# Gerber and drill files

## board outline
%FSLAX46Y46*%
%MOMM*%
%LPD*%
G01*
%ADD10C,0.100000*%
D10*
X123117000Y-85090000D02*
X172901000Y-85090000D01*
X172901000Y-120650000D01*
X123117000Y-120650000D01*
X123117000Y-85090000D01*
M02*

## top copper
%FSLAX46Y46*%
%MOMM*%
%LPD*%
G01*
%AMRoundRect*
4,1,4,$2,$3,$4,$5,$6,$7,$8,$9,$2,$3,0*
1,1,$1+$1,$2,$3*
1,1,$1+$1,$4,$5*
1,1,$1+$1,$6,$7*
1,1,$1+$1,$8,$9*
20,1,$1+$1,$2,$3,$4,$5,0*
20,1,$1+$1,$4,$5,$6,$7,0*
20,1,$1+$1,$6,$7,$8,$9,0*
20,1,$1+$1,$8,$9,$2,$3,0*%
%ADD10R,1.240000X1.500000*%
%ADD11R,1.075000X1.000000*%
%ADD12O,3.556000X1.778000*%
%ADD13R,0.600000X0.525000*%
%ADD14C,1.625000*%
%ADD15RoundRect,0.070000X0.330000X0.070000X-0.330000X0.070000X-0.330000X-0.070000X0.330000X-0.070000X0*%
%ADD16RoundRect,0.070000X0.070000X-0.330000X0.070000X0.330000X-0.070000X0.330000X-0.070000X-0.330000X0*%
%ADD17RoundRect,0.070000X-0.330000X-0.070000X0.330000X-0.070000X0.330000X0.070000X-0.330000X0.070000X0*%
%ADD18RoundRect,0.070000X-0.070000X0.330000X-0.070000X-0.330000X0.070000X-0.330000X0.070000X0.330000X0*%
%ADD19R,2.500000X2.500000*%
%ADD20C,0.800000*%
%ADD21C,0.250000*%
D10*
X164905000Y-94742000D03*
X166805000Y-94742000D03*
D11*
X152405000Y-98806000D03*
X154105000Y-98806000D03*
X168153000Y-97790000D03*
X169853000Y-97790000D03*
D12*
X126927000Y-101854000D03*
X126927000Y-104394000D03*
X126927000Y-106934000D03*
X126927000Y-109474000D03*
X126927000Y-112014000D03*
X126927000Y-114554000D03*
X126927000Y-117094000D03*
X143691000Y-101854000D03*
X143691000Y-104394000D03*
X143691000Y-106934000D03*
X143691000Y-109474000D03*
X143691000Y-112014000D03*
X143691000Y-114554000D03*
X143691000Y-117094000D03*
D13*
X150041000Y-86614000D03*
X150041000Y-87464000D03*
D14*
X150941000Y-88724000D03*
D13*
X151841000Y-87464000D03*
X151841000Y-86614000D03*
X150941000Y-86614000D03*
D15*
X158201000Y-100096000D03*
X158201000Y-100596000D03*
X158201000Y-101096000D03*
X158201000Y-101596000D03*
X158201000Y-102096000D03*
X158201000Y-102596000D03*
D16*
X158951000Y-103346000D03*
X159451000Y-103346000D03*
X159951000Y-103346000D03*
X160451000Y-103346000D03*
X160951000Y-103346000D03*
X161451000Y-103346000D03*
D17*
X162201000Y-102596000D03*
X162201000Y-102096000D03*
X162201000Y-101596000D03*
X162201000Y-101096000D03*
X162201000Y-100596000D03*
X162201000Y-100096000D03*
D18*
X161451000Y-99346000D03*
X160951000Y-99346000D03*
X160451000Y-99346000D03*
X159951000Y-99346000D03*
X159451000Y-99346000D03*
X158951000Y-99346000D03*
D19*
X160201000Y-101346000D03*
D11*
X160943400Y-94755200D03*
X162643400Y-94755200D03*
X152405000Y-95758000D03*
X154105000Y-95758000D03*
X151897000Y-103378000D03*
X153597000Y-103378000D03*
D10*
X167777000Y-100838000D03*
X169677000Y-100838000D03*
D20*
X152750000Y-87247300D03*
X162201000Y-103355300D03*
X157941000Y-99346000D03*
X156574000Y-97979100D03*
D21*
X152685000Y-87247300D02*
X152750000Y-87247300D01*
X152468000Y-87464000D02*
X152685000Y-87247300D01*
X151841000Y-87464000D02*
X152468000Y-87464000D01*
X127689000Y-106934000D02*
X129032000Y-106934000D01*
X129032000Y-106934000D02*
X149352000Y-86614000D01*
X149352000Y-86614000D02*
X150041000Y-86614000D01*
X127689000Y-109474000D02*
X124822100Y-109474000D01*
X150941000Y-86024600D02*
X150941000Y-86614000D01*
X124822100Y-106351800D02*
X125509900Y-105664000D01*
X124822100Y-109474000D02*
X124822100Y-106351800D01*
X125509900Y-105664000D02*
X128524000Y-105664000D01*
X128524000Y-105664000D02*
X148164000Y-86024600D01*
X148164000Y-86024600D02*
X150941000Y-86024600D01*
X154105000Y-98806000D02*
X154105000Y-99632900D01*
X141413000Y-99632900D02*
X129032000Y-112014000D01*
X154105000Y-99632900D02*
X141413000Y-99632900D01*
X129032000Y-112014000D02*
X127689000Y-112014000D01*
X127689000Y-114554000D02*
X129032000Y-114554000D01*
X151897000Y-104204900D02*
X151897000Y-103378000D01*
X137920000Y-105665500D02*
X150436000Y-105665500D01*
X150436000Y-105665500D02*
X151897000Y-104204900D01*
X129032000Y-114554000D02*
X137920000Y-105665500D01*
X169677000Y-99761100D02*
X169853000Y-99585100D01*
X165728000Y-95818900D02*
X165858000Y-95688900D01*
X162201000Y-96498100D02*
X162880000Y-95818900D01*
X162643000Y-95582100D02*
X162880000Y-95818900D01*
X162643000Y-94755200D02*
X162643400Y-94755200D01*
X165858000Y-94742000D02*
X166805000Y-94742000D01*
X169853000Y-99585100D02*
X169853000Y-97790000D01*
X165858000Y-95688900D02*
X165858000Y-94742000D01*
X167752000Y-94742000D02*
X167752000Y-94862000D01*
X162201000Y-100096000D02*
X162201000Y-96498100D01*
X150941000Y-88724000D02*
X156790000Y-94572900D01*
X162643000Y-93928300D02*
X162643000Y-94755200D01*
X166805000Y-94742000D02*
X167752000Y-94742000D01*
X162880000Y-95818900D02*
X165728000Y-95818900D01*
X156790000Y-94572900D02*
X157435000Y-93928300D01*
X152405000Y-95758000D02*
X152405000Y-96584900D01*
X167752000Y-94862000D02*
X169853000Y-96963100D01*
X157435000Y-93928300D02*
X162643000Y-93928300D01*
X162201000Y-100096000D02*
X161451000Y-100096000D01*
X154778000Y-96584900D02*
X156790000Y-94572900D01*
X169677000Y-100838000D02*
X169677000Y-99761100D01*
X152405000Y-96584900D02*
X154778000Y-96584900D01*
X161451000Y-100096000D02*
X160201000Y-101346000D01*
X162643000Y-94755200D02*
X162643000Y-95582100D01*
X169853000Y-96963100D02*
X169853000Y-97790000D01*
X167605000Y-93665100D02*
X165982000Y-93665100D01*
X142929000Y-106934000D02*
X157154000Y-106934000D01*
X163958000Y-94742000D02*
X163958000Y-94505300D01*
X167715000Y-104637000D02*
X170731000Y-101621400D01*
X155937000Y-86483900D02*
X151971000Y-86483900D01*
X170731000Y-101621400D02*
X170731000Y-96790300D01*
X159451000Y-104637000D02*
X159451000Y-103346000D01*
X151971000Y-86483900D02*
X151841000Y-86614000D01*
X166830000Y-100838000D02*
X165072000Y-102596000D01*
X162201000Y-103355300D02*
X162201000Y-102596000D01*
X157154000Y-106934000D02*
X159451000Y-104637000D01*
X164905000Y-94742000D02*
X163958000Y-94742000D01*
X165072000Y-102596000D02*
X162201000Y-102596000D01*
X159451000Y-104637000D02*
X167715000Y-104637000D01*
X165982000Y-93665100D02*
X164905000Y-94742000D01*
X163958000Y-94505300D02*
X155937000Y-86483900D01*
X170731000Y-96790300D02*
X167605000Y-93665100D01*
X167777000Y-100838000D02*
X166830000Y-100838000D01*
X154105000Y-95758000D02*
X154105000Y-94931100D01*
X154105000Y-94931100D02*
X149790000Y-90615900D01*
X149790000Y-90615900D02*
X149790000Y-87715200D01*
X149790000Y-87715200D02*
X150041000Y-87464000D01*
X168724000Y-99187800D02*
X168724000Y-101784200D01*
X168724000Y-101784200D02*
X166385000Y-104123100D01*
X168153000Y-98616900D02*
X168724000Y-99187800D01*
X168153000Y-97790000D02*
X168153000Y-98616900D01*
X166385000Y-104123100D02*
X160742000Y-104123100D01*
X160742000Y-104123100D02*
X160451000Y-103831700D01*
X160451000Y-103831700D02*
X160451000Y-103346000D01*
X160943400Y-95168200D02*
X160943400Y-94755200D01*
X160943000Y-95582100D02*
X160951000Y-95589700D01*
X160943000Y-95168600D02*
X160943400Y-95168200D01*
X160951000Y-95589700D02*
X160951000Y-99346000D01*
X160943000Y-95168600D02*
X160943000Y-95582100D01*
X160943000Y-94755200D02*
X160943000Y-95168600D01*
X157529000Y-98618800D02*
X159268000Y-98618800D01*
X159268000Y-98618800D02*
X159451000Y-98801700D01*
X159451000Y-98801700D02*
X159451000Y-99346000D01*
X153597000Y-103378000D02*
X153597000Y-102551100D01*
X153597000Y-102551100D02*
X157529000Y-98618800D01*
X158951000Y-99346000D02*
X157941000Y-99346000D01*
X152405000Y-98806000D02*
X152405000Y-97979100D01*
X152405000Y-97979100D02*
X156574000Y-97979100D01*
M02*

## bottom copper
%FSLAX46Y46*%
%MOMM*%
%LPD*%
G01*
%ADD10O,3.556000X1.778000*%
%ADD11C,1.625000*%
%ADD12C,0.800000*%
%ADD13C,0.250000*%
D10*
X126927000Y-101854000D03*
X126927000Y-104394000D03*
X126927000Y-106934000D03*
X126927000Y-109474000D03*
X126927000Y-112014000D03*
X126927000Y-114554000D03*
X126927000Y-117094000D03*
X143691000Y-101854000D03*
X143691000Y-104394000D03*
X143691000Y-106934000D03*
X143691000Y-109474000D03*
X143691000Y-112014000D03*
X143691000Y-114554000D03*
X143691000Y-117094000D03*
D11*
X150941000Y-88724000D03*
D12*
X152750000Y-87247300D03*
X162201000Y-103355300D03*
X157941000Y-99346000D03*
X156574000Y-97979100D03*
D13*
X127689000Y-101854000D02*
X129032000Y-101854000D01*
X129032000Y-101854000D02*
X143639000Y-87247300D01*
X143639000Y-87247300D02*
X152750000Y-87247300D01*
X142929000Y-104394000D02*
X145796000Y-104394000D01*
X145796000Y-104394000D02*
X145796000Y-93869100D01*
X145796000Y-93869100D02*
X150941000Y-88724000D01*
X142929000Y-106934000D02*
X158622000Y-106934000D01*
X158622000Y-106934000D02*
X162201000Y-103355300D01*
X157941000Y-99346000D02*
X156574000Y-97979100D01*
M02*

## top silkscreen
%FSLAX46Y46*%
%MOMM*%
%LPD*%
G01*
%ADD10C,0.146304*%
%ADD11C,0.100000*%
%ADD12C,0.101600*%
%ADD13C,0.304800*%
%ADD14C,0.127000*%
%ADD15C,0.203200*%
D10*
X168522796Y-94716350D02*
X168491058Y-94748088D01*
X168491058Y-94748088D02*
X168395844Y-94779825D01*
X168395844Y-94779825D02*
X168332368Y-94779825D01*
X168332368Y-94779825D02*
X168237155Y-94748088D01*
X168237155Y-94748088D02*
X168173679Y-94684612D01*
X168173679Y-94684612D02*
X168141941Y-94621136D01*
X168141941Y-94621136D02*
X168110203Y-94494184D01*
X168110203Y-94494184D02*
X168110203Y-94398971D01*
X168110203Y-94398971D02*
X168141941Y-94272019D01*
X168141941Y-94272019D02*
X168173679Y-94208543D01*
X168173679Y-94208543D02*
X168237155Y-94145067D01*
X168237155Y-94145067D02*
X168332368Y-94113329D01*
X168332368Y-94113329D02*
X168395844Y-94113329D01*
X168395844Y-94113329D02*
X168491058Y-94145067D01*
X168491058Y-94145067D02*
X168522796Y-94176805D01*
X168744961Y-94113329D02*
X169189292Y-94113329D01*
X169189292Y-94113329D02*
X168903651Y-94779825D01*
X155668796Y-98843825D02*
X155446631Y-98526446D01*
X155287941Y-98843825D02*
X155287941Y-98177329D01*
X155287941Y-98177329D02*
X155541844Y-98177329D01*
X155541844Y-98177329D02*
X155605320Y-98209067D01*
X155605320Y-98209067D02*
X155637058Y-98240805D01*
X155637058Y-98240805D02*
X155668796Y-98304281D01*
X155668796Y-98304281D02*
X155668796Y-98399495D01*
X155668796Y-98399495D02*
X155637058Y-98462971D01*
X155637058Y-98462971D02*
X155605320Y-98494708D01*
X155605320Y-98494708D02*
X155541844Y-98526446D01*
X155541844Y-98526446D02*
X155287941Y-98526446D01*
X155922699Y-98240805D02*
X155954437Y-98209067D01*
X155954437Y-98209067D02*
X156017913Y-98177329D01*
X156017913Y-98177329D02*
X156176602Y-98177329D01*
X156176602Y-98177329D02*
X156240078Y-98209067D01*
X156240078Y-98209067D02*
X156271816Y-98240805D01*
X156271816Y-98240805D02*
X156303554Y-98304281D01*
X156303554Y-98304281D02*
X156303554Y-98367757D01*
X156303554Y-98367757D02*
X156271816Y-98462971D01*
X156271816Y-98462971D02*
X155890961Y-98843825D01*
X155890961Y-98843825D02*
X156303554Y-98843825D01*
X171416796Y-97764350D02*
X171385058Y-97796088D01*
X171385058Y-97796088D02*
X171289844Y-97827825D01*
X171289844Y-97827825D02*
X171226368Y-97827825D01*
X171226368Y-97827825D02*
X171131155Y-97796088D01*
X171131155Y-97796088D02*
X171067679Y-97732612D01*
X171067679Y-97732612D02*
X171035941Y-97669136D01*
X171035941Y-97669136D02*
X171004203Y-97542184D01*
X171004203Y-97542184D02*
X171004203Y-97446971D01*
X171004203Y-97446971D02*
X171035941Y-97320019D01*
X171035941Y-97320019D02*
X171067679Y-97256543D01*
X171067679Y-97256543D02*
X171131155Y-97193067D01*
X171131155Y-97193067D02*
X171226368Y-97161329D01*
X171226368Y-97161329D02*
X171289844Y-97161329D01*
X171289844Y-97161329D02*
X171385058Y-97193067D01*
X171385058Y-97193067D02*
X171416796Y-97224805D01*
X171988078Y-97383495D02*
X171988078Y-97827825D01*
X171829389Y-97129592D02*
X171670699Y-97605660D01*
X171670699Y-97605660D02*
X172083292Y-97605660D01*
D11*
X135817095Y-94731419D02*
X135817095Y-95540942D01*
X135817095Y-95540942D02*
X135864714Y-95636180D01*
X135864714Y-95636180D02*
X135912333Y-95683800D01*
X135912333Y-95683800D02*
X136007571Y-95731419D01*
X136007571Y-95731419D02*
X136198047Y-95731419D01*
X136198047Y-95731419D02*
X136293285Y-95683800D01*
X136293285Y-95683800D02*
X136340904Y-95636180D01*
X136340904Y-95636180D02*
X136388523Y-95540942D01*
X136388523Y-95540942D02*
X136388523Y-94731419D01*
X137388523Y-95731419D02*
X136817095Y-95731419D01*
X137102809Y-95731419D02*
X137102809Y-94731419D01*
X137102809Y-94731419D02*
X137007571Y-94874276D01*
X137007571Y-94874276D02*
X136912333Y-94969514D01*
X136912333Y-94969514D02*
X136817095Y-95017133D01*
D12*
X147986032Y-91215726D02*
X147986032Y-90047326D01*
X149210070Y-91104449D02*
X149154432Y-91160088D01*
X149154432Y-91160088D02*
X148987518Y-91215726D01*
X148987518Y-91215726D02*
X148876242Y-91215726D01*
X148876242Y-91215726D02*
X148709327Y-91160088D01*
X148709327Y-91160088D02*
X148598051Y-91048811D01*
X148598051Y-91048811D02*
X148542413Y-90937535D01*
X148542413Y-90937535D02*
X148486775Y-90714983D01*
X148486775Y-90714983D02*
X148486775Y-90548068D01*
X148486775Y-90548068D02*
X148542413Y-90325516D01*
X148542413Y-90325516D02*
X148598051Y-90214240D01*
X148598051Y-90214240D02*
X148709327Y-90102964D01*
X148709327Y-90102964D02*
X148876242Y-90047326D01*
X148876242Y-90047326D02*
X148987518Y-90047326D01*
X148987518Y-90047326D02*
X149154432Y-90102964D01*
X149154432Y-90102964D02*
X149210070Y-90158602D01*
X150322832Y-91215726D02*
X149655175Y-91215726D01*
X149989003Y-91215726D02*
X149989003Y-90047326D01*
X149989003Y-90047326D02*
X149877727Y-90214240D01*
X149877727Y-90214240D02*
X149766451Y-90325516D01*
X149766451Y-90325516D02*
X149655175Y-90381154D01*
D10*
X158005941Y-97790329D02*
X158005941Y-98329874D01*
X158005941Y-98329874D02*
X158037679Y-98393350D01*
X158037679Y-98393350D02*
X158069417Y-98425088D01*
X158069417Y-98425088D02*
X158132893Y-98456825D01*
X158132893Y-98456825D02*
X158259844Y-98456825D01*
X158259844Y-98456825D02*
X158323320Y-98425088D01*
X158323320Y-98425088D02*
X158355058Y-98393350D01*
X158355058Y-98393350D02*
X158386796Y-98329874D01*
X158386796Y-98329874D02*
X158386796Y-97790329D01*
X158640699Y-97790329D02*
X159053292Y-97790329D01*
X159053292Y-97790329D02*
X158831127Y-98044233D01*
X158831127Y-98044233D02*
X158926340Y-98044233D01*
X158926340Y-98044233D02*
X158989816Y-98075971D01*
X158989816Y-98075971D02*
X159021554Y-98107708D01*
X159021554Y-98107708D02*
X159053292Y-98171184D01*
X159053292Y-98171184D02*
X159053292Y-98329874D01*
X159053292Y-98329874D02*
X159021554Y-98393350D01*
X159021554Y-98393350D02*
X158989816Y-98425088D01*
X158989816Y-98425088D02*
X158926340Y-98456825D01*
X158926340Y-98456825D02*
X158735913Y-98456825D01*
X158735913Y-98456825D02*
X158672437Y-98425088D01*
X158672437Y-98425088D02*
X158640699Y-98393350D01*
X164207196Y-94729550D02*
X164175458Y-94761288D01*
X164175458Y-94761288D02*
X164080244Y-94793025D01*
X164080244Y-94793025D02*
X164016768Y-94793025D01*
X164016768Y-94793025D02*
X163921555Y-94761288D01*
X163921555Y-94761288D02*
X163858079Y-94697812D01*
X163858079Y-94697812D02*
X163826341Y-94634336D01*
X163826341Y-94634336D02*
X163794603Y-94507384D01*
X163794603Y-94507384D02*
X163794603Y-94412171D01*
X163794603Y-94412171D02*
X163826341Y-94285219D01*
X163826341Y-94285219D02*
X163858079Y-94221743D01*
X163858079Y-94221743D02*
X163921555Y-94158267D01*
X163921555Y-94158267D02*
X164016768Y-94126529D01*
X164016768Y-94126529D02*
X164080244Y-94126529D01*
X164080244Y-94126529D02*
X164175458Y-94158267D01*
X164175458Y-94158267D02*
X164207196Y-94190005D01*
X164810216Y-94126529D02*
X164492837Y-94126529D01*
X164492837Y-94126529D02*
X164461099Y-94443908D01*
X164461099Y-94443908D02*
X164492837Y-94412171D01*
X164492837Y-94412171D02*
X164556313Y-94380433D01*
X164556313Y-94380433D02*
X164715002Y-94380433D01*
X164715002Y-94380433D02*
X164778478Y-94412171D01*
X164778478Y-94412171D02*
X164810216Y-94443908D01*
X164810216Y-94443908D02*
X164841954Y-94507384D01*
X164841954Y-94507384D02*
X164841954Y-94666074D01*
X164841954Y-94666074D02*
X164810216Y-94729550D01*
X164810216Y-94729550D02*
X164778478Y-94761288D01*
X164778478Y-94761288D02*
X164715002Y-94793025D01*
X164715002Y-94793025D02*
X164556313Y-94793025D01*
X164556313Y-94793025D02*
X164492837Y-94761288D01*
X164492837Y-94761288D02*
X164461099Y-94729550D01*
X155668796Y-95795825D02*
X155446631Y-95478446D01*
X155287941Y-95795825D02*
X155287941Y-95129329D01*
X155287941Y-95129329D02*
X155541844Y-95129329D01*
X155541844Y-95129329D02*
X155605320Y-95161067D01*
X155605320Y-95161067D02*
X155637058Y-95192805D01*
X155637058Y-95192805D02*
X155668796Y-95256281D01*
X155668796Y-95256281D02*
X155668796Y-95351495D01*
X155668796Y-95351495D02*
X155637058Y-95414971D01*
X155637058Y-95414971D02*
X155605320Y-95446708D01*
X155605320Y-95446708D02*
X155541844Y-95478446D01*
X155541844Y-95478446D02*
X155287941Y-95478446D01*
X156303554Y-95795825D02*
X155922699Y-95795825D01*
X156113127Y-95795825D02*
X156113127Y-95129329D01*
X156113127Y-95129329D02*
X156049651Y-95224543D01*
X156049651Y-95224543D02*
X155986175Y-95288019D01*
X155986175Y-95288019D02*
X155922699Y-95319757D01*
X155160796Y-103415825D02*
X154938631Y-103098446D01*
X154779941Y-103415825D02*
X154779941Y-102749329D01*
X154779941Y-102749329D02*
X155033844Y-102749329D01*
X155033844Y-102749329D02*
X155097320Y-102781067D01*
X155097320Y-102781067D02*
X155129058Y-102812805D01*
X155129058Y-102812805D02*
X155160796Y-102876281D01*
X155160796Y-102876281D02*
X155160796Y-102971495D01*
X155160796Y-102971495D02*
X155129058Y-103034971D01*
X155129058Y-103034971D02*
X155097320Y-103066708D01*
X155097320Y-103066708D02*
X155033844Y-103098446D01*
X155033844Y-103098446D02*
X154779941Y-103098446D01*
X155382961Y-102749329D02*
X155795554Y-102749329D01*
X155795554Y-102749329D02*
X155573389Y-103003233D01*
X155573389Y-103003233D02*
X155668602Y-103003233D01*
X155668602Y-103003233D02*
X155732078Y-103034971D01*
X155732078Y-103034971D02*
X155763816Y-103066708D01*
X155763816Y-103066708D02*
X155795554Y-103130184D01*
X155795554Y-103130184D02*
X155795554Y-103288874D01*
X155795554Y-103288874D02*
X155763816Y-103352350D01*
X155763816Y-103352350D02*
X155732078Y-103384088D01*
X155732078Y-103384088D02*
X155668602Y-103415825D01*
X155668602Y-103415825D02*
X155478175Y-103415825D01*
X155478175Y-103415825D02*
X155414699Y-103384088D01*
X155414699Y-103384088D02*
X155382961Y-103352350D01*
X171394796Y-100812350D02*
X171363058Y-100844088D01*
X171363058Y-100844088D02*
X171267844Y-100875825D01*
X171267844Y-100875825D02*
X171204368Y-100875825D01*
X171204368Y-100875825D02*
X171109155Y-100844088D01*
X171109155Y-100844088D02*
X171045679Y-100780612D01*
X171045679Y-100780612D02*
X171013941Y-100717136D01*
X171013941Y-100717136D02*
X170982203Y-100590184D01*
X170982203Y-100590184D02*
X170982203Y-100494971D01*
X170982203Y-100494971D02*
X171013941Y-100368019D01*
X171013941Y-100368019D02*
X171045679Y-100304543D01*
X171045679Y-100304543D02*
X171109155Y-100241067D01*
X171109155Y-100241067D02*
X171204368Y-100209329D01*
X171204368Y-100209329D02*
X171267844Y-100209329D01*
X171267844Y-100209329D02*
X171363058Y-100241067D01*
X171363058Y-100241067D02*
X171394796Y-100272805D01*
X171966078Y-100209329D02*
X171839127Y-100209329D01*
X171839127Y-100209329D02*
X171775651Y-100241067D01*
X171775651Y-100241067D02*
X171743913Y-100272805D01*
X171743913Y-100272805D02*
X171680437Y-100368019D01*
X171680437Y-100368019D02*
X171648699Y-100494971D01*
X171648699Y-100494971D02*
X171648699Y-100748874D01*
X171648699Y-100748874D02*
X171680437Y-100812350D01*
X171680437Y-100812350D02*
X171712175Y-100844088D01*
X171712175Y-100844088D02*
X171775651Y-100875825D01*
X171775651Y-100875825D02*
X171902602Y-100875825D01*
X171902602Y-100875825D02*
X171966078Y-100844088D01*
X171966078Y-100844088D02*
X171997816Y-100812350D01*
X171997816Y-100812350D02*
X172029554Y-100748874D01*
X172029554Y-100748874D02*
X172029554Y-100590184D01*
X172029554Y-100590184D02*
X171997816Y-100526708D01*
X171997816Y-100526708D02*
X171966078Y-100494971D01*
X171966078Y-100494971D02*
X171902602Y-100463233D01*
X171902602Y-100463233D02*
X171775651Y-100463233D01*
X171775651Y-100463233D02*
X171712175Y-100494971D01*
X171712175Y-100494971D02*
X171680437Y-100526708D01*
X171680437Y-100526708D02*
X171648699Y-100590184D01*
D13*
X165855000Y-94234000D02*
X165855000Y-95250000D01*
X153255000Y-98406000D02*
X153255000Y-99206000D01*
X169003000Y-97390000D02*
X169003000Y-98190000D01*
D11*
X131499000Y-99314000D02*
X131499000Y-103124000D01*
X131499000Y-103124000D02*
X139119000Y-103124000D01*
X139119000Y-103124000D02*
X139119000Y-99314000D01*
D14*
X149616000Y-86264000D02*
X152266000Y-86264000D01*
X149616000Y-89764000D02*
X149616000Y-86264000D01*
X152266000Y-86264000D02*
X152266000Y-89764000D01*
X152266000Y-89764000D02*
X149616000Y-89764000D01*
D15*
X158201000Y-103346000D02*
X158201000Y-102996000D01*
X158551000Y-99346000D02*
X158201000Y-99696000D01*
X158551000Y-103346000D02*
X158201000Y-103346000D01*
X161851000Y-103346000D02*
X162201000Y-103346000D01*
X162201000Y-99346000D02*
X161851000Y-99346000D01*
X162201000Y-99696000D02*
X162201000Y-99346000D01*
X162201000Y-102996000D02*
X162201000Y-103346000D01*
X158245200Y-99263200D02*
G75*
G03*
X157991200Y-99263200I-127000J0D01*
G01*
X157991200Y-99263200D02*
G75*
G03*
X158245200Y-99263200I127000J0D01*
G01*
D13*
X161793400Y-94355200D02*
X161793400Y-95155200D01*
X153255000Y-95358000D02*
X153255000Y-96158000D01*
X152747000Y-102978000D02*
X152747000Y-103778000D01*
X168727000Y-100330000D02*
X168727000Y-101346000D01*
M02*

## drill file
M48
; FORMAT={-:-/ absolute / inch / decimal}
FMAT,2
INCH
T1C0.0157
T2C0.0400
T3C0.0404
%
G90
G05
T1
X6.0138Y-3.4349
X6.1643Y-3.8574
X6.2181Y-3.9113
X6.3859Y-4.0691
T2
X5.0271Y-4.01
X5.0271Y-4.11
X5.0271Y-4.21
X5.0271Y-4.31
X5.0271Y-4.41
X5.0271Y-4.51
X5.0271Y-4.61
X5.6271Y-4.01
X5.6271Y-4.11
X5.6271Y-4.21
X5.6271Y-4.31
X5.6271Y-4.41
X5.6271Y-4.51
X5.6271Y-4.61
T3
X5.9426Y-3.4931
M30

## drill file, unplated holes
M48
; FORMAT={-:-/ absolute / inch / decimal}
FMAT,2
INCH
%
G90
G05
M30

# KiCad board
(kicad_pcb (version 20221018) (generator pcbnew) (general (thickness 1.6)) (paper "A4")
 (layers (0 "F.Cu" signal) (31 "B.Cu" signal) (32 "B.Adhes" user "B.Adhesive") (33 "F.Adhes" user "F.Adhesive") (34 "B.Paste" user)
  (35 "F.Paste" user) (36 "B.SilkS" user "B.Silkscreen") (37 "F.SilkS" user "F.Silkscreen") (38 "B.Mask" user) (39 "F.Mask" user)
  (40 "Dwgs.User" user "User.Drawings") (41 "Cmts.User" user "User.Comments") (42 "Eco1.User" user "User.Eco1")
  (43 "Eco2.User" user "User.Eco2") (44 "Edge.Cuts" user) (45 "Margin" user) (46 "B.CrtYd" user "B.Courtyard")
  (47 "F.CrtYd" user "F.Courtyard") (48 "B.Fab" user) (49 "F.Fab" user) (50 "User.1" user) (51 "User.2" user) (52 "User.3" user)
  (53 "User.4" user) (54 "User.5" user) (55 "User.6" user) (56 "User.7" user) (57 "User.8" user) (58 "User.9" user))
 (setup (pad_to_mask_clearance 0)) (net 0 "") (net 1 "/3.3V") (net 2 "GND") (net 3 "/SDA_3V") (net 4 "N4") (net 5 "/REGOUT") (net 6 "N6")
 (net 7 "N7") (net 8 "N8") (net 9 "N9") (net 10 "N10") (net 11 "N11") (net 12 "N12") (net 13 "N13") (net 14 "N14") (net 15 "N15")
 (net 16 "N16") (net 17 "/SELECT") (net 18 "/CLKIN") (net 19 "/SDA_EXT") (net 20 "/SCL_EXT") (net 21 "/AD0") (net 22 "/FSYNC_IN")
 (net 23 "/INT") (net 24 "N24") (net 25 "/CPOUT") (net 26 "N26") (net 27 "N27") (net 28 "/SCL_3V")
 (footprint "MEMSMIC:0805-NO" (layer "F.Cu") (at 165.855 94.742)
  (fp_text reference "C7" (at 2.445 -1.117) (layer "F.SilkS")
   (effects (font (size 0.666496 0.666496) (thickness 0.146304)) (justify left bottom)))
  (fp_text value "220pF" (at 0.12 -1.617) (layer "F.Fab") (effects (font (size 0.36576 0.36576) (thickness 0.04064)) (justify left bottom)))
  (fp_line (start 0 -0.508) (end 0 0.508) (stroke (width 0.3048) (type solid)) (layer "F.SilkS"))
  (pad "1" smd rect (at -0.95 0) (size 1.24 1.5) (layers "F.Cu" "F.Paste" "F.Mask") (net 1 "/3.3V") (solder_mask_margin 0.0508)
   (thermal_bridge_angle 0))
  (pad "2" smd rect (at 0.95 0) (size 1.24 1.5) (layers "F.Cu" "F.Paste" "F.Mask") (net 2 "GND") (solder_mask_margin 0.0508)
   (thermal_bridge_angle 0)))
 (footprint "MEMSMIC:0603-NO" (layer "F.Cu") (at 153.255 98.806)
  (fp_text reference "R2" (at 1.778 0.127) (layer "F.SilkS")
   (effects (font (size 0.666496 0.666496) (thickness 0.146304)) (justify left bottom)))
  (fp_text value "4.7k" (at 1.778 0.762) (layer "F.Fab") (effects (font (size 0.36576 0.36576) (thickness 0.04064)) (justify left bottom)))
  (fp_line (start 0 -0.4) (end 0 0.4) (stroke (width 0.3048) (type solid)) (layer "F.SilkS"))
  (pad "1" smd rect (at -0.85 0) (size 1.075 1) (layers "F.Cu" "F.Paste" "F.Mask") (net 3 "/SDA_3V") (solder_mask_margin 0.0508)
   (thermal_bridge_angle 0))
  (pad "2" smd rect (at 0.85 0) (size 1.075 1) (layers "F.Cu" "F.Paste" "F.Mask") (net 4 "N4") (solder_mask_margin 0.0508)
   (thermal_bridge_angle 0)))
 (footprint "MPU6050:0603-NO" (layer "F.Cu") (at 169.003 97.79)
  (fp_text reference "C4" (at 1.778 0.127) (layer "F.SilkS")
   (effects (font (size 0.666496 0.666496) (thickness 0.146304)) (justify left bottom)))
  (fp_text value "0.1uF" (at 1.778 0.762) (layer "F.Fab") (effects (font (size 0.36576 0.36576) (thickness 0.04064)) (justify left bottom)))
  (fp_line (start 0 -0.4) (end 0 0.4) (stroke (width 0.3048) (type solid)) (layer "F.SilkS"))
  (pad "1" smd rect (at -0.85 0) (size 1.075 1) (layers "F.Cu" "F.Paste" "F.Mask") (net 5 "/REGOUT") (solder_mask_margin 0.0508)
   (thermal_bridge_angle 0))
  (pad "2" smd rect (at 0.85 0) (size 1.075 1) (layers "F.Cu" "F.Paste" "F.Mask") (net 2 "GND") (solder_mask_margin 0.0508)
   (thermal_bridge_angle 0)))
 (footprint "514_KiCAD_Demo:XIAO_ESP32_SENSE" (layer "F.Cu") (at 135.309 109.474)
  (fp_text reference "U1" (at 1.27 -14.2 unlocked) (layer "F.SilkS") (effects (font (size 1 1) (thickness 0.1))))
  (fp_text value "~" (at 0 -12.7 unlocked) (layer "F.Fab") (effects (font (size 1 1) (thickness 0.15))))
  (fp_line (start -3.81 -10.16) (end -3.81 -6.35) (stroke (width 0.1) (type default)) (layer "F.SilkS"))
  (fp_line (start -3.81 -6.35) (end 3.81 -6.35) (stroke (width 0.1) (type default)) (layer "F.SilkS"))
  (fp_line (start 3.81 -6.35) (end 3.81 -10.16) (stroke (width 0.1) (type default)) (layer "F.SilkS"))
  (pad "1" thru_hole oval (at -7.62 -7.62) (size 3.556 1.778) (drill 1.016 (offset -0.762 0)) (layers "*.Cu" "*.Mask") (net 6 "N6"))
  (pad "2" thru_hole oval (at -7.62 -5.08) (size 3.556 1.778) (drill 1.016 (offset -0.762 0)) (layers "*.Cu" "*.Mask") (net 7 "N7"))
  (pad "3" thru_hole oval (at -7.62 -2.54) (size 3.556 1.778) (drill 1.016 (offset -0.762 0)) (layers "*.Cu" "*.Mask") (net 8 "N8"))
  (pad "4" thru_hole oval (at -7.62 0) (size 3.556 1.778) (drill 1.016 (offset -0.762 0)) (layers "*.Cu" "*.Mask") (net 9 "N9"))
  (pad "5" thru_hole oval (at -7.62 2.54) (size 3.556 1.778) (drill 1.016 (offset -0.762 0)) (layers "*.Cu" "*.Mask") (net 4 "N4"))
  (pad "6" thru_hole oval (at -7.62 5.08) (size 3.556 1.778) (drill 1.016 (offset -0.762 0)) (layers "*.Cu" "*.Mask") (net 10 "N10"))
  (pad "7" thru_hole oval (at -7.62 7.62) (size 3.556 1.778) (drill 1.016 (offset -0.762 0)) (layers "*.Cu" "*.Mask") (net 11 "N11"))
  (pad "8" thru_hole oval (at 7.62 -7.62) (size 3.556 1.778) (drill 1.016 (offset 0.762 0)) (layers "*.Cu" "*.Mask") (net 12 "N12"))
  (pad "9" thru_hole oval (at 7.62 -5.08) (size 3.556 1.778) (drill 1.016 (offset 0.762 0)) (layers "*.Cu" "*.Mask") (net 2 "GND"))
  (pad "10" thru_hole oval (at 7.62 -2.54) (size 3.556 1.778) (drill 1.016 (offset 0.762 0)) (layers "*.Cu" "*.Mask") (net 1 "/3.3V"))
  (pad "11" thru_hole oval (at 7.62 0) (size 3.556 1.778) (drill 1.016 (offset 0.762 0)) (layers "*.Cu" "*.Mask") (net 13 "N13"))
  (pad "12" thru_hole oval (at 7.62 2.54) (size 3.556 1.778) (drill 1.016 (offset 0.762 0)) (layers "*.Cu" "*.Mask") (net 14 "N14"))
  (pad "13" thru_hole oval (at 7.62 5.08) (size 3.556 1.778) (drill 1.016 (offset 0.762 0)) (layers "*.Cu" "*.Mask") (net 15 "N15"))
  (pad "14" thru_hole oval (at 7.62 7.62) (size 3.556 1.778) (drill 1.016 (offset 0.762 0)) (layers "*.Cu" "*.Mask") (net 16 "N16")))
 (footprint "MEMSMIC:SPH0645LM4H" (layer "F.Cu") (at 150.941 88.014)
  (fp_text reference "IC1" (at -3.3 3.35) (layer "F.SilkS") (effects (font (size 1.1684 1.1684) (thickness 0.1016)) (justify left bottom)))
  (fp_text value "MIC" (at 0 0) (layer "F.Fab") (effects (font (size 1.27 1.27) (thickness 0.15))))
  (fp_line (start -1.325 -1.75) (end 1.325 -1.75) (stroke (width 0.127) (type solid)) (layer "F.SilkS"))
  (fp_line (start -1.325 1.75) (end -1.325 -1.75) (stroke (width 0.127) (type solid)) (layer "F.SilkS"))
  (fp_line (start 1.325 -1.75) (end 1.325 1.75) (stroke (width 0.127) (type solid)) (layer "F.SilkS"))
  (fp_line (start 1.325 1.75) (end -1.325 1.75) (stroke (width 0.127) (type solid)) (layer "F.SilkS"))
  (pad "1" smd rect (at -0.9 -1.4) (size 0.6 0.525) (layers "F.Cu" "F.Paste" "F.Mask") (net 8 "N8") (solder_mask_margin 0.0508)
   (thermal_bridge_angle 0))
  (pad "2" smd rect (at -0.9 -0.55) (size 0.6 0.525) (layers "F.Cu" "F.Paste" "F.Mask") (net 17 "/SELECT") (solder_mask_margin 0.0508)
   (thermal_bridge_angle 0))
  (pad "3" thru_hole circle (at 0 0.71) (size 1.625 1.625) (drill 1.025) (layers "*.Cu" "*.Mask") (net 2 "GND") (solder_mask_margin 0.0508)
   (thermal_bridge_angle 0))
  (pad "4" smd rect (at 0.9 -0.55) (size 0.6 0.525) (layers "F.Cu" "F.Paste" "F.Mask") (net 6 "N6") (solder_mask_margin 0.0508)
   (thermal_bridge_angle 0))
  (pad "5" smd rect (at 0.9 -1.4) (size 0.6 0.525) (layers "F.Cu" "F.Paste" "F.Mask") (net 1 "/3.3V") (solder_mask_margin 0.0508)
   (thermal_bridge_angle 0))
  (pad "6" smd rect (at 0 -1.4) (size 0.6 0.525) (layers "F.Cu" "F.Paste" "F.Mask") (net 9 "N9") (solder_mask_margin 0.0508)
   (thermal_bridge_angle 0)))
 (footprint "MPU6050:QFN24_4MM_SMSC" (layer "F.Cu") (at 160.201 101.346)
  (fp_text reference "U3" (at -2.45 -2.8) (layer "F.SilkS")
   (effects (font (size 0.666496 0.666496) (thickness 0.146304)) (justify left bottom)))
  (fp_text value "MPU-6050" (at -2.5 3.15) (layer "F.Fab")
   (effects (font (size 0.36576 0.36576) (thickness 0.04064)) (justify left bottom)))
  (fp_line (start -2 2) (end -2 1.65) (stroke (width 0.2032) (type solid)) (layer "F.SilkS"))
  (fp_line (start -1.65 -2) (end -2 -1.65) (stroke (width 0.2032) (type solid)) (layer "F.SilkS"))
  (fp_line (start -1.65 2) (end -2 2) (stroke (width 0.2032) (type solid)) (layer "F.SilkS"))
  (fp_line (start 1.65 2) (end 2 2) (stroke (width 0.2032) (type solid)) (layer "F.SilkS"))
  (fp_line (start 2 -2) (end 1.65 -2) (stroke (width 0.2032) (type solid)) (layer "F.SilkS"))
  (fp_line (start 2 -1.65) (end 2 -2) (stroke (width 0.2032) (type solid)) (layer "F.SilkS"))
  (fp_line (start 2 1.65) (end 2 2) (stroke (width 0.2032) (type solid)) (layer "F.SilkS"))
  (fp_circle (center -2.0828 -2.0828) (end -1.9558 -2.0828) (stroke (width 0.2032) (type solid)) (fill none) (layer "F.SilkS"))
  (pad "1" smd roundrect (at -2 -1.25 180) (size 0.8 0.28) (layers "F.Cu" "F.Paste" "F.Mask") (roundrect_rratio 0.25) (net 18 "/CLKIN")
   (solder_mask_margin 0.0508) (thermal_bridge_angle 0))
  (pad "2" smd roundrect (at -2 -0.75 180) (size 0.8 0.28) (layers "F.Cu" "F.Paste" "F.Mask") (roundrect_rratio 0.25)
   (solder_mask_margin 0.0508) (thermal_bridge_angle 0))
  (pad "3" smd roundrect (at -2 -0.25 180) (size 0.8 0.28) (layers "F.Cu" "F.Paste" "F.Mask") (roundrect_rratio 0.25)
   (solder_mask_margin 0.0508) (thermal_bridge_angle 0))
  (pad "4" smd roundrect (at -2 0.25 180) (size 0.8 0.28) (layers "F.Cu" "F.Paste" "F.Mask") (roundrect_rratio 0.25)
   (solder_mask_margin 0.0508) (thermal_bridge_angle 0))
  (pad "5" smd roundrect (at -2 0.75 180) (size 0.8 0.28) (layers "F.Cu" "F.Paste" "F.Mask") (roundrect_rratio 0.25)
   (solder_mask_margin 0.0508) (thermal_bridge_angle 0))
  (pad "6" smd roundrect (at -2 1.25 180) (size 0.8 0.28) (layers "F.Cu" "F.Paste" "F.Mask") (roundrect_rratio 0.25) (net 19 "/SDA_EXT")
   (solder_mask_margin 0.0508) (thermal_bridge_angle 0))
  (pad "7" smd roundrect (at -1.25 2 90) (size 0.8 0.28) (layers "F.Cu" "F.Paste" "F.Mask") (roundrect_rratio 0.25) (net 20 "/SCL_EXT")
   (solder_mask_margin 0.0508) (thermal_bridge_angle 0))
  (pad "8" smd roundrect (at -0.75 2 90) (size 0.8 0.28) (layers "F.Cu" "F.Paste" "F.Mask") (roundrect_rratio 0.25) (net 1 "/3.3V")
   (solder_mask_margin 0.0508) (thermal_bridge_angle 0))
  (pad "9" smd roundrect (at -0.25 2 90) (size 0.8 0.28) (layers "F.Cu" "F.Paste" "F.Mask") (roundrect_rratio 0.25) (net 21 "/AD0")
   (solder_mask_margin 0.0508) (thermal_bridge_angle 0))
  (pad "10" smd roundrect (at 0.25 2 90) (size 0.8 0.28) (layers "F.Cu" "F.Paste" "F.Mask") (roundrect_rratio 0.25) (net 5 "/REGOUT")
   (solder_mask_margin 0.0508) (thermal_bridge_angle 0))
  (pad "11" smd roundrect (at 0.75 2 90) (size 0.8 0.28) (layers "F.Cu" "F.Paste" "F.Mask") (roundrect_rratio 0.25) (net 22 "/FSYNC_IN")
   (solder_mask_margin 0.0508) (thermal_bridge_angle 0))
  (pad "12" smd roundrect (at 1.25 2 90) (size 0.8 0.28) (layers "F.Cu" "F.Paste" "F.Mask") (roundrect_rratio 0.25) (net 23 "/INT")
   (solder_mask_margin 0.0508) (thermal_bridge_angle 0))
  (pad "13" smd roundrect (at 2 1.25) (size 0.8 0.28) (layers "F.Cu" "F.Paste" "F.Mask") (roundrect_rratio 0.25) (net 1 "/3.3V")
   (solder_mask_margin 0.0508) (thermal_bridge_angle 0))
  (pad "14" smd roundrect (at 2 0.75) (size 0.8 0.28) (layers "F.Cu" "F.Paste" "F.Mask") (roundrect_rratio 0.25) (solder_mask_margin 0.0508)
   (thermal_bridge_angle 0))
  (pad "15" smd roundrect (at 2 0.25) (size 0.8 0.28) (layers "F.Cu" "F.Paste" "F.Mask") (roundrect_rratio 0.25) (solder_mask_margin 0.0508)
   (thermal_bridge_angle 0))
  (pad "16" smd roundrect (at 2 -0.25) (size 0.8 0.28) (layers "F.Cu" "F.Paste" "F.Mask") (roundrect_rratio 0.25)
   (solder_mask_margin 0.0508) (thermal_bridge_angle 0))
  (pad "17" smd roundrect (at 2 -0.75) (size 0.8 0.28) (layers "F.Cu" "F.Paste" "F.Mask") (roundrect_rratio 0.25)
   (solder_mask_margin 0.0508) (thermal_bridge_angle 0))
  (pad "18" smd roundrect (at 2 -1.25) (size 0.8 0.28) (layers "F.Cu" "F.Paste" "F.Mask") (roundrect_rratio 0.25) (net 2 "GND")
   (solder_mask_margin 0.0508) (thermal_bridge_angle 0))
  (pad "19" smd roundrect (at 1.25 -2 270) (size 0.8 0.28) (layers "F.Cu" "F.Paste" "F.Mask") (roundrect_rratio 0.25) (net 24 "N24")
   (solder_mask_margin 0.0508) (thermal_bridge_angle 0))
  (pad "20" smd roundrect (at 0.75 -2 270) (size 0.8 0.28) (layers "F.Cu" "F.Paste" "F.Mask") (roundrect_rratio 0.25) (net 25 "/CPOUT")
   (solder_mask_margin 0.0508) (thermal_bridge_angle 0))
  (pad "21" smd roundrect (at 0.25 -2 270) (size 0.8 0.28) (layers "F.Cu" "F.Paste" "F.Mask") (roundrect_rratio 0.25) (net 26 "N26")
   (solder_mask_margin 0.0508) (thermal_bridge_angle 0))
  (pad "22" smd roundrect (at -0.25 -2 270) (size 0.8 0.28) (layers "F.Cu" "F.Paste" "F.Mask") (roundrect_rratio 0.25) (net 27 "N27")
   (solder_mask_margin 0.0508) (thermal_bridge_angle 0))
  (pad "23" smd roundrect (at -0.75 -2 270) (size 0.8 0.28) (layers "F.Cu" "F.Paste" "F.Mask") (roundrect_rratio 0.25) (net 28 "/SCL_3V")
   (solder_mask_margin 0.0508) (thermal_bridge_angle 0))
  (pad "24" smd roundrect (at -1.25 -2 270) (size 0.8 0.28) (layers "F.Cu" "F.Paste" "F.Mask") (roundrect_rratio 0.25) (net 3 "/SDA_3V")
   (solder_mask_margin 0.0508) (thermal_bridge_angle 0))
  (pad "THERM" smd rect (at 0 0) (size 2.5 2.5) (layers "F.Cu" "F.Mask") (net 2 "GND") (solder_mask_margin 0.0508) (thermal_bridge_angle 0)))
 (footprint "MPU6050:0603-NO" (layer "F.Cu") (at 161.7934 94.7552)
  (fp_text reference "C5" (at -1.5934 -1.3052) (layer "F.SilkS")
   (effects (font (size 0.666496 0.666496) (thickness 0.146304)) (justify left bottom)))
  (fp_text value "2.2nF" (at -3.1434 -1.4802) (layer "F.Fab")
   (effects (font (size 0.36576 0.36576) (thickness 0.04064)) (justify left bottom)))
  (fp_line (start 0 -0.4) (end 0 0.4) (stroke (width 0.3048) (type solid)) (layer "F.SilkS"))
  (pad "1" smd rect (at -0.85 0) (size 1.075 1) (layers "F.Cu" "F.Paste" "F.Mask") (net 25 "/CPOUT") (solder_mask_margin 0.0508)
   (thermal_bridge_angle 0))
  (pad "2" smd rect (at 0.85 0) (size 1.075 1) (layers "F.Cu" "F.Paste" "F.Mask") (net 2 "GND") (solder_mask_margin 0.0508)
   (thermal_bridge_angle 0)))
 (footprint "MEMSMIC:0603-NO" (layer "F.Cu") (at 153.255 95.758)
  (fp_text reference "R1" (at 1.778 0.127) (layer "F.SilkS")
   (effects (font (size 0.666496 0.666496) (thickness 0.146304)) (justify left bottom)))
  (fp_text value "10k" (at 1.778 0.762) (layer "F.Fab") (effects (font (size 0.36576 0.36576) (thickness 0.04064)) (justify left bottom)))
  (fp_line (start 0 -0.4) (end 0 0.4) (stroke (width 0.3048) (type solid)) (layer "F.SilkS"))
  (pad "1" smd rect (at -0.85 0) (size 1.075 1) (layers "F.Cu" "F.Paste" "F.Mask") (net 2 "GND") (solder_mask_margin 0.0508)
   (thermal_bridge_angle 0))
  (pad "2" smd rect (at 0.85 0) (size 1.075 1) (layers "F.Cu" "F.Paste" "F.Mask") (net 17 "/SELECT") (solder_mask_margin 0.0508)
   (thermal_bridge_angle 0)))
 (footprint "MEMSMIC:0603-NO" (layer "F.Cu") (at 152.747 103.378)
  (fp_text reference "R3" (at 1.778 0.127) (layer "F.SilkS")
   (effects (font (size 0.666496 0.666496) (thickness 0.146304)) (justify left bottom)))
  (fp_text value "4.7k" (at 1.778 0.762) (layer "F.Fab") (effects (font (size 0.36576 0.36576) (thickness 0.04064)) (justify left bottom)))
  (fp_line (start 0 -0.4) (end 0 0.4) (stroke (width 0.3048) (type solid)) (layer "F.SilkS"))
  (pad "1" smd rect (at -0.85 0) (size 1.075 1) (layers "F.Cu" "F.Paste" "F.Mask") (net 10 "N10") (solder_mask_margin 0.0508)
   (thermal_bridge_angle 0))
  (pad "2" smd rect (at 0.85 0) (size 1.075 1) (layers "F.Cu" "F.Paste" "F.Mask") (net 28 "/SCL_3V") (solder_mask_margin 0.0508)
   (thermal_bridge_angle 0)))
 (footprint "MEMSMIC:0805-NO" (layer "F.Cu") (at 168.727 100.838)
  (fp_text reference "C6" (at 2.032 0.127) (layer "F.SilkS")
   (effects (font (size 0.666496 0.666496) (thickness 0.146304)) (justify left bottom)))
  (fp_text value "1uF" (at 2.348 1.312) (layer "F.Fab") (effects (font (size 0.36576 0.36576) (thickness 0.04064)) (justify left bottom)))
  (fp_line (start 0 -0.508) (end 0 0.508) (stroke (width 0.3048) (type solid)) (layer "F.SilkS"))
  (pad "1" smd rect (at -0.95 0) (size 1.24 1.5) (layers "F.Cu" "F.Paste" "F.Mask") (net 1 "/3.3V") (solder_mask_margin 0.0508)
   (thermal_bridge_angle 0))
  (pad "2" smd rect (at 0.95 0) (size 1.24 1.5) (layers "F.Cu" "F.Paste" "F.Mask") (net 2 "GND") (solder_mask_margin 0.0508)
   (thermal_bridge_angle 0)))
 (gr_rect (start 123.117 85.09) (end 172.901 120.65) (stroke (width 0.1) (type default)) (fill none) (layer "Edge.Cuts"))
 (segment (start 152.685 87.2473) (end 152.75 87.2473) (width 0.25) (layer "F.Cu") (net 6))
 (segment (start 152.468 87.464) (end 152.685 87.2473) (width 0.25) (layer "F.Cu") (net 6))
 (segment (start 151.841 87.464) (end 152.468 87.464) (width 0.25) (layer "F.Cu") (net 6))
 (via (at 152.75 87.2473) (size 0.8) (drill 0.4) (layers "F.Cu" "B.Cu") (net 6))
 (segment (start 127.689 101.854) (end 129.032 101.854) (width 0.25) (layer "B.Cu") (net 6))
 (segment (start 129.032 101.854) (end 143.639 87.2473) (width 0.25) (layer "B.Cu") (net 6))
 (segment (start 143.639 87.2473) (end 152.75 87.2473) (width 0.25) (layer "B.Cu") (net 6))
 (segment (start 127.689 106.934) (end 129.032 106.934) (width 0.25) (layer "F.Cu") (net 8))
 (segment (start 129.032 106.934) (end 149.352 86.614) (width 0.25) (layer "F.Cu") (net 8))
 (segment (start 149.352 86.614) (end 150.041 86.614) (width 0.25) (layer "F.Cu") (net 8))
 (segment (start 127.689 109.474) (end 124.8221 109.474) (width 0.25) (layer "F.Cu") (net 9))
 (segment (start 150.941 86.0246) (end 150.941 86.614) (width 0.25) (layer "F.Cu") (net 9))
 (segment (start 124.8221 106.3518) (end 125.5099 105.664) (width 0.25) (layer "F.Cu") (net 9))
 (segment (start 124.8221 109.474) (end 124.8221 106.3518) (width 0.25) (layer "F.Cu") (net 9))
 (segment (start 125.5099 105.664) (end 128.524 105.664) (width 0.25) (layer "F.Cu") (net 9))
 (segment (start 128.524 105.664) (end 148.164 86.0246) (width 0.25) (layer "F.Cu") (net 9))
 (segment (start 148.164 86.0246) (end 150.941 86.0246) (width 0.25) (layer "F.Cu") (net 9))
 (segment (start 154.105 98.806) (end 154.105 99.6329) (width 0.25) (layer "F.Cu") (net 4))
 (segment (start 141.413 99.6329) (end 129.032 112.014) (width 0.25) (layer "F.Cu") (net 4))
 (segment (start 154.105 99.6329) (end 141.413 99.6329) (width 0.25) (layer "F.Cu") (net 4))
 (segment (start 129.032 112.014) (end 127.689 112.014) (width 0.25) (layer "F.Cu") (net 4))
 (segment (start 127.689 114.554) (end 129.032 114.554) (width 0.25) (layer "F.Cu") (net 10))
 (segment (start 151.897 104.2049) (end 151.897 103.378) (width 0.25) (layer "F.Cu") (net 10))
 (segment (start 137.92 105.6655) (end 150.436 105.6655) (width 0.25) (layer "F.Cu") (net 10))
 (segment (start 150.436 105.6655) (end 151.897 104.2049) (width 0.25) (layer "F.Cu") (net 10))
 (segment (start 129.032 114.554) (end 137.92 105.6655) (width 0.25) (layer "F.Cu") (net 10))
 (segment (start 169.677 99.7611) (end 169.853 99.5851) (width 0.25) (layer "F.Cu") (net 2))
 (segment (start 165.728 95.8189) (end 165.858 95.6889) (width 0.25) (layer "F.Cu") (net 2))
 (segment (start 162.201 96.4981) (end 162.88 95.8189) (width 0.25) (layer "F.Cu") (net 2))
 (segment (start 162.643 95.5821) (end 162.88 95.8189) (width 0.25) (layer "F.Cu") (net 2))
 (segment (start 162.643 94.7552) (end 162.6434 94.7552) (width 0.25) (layer "F.Cu") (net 2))
 (segment (start 165.858 94.742) (end 166.805 94.742) (width 0.25) (layer "F.Cu") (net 2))
 (segment (start 169.853 99.5851) (end 169.853 97.79) (width 0.25) (layer "F.Cu") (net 2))
 (segment (start 165.858 95.6889) (end 165.858 94.742) (width 0.25) (layer "F.Cu") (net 2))
 (segment (start 167.752 94.742) (end 167.752 94.862) (width 0.25) (layer "F.Cu") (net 2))
 (segment (start 162.201 100.096) (end 162.201 96.4981) (width 0.25) (layer "F.Cu") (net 2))
 (segment (start 150.941 88.724) (end 156.79 94.5729) (width 0.25) (layer "F.Cu") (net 2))
 (segment (start 162.643 93.9283) (end 162.643 94.7552) (width 0.25) (layer "F.Cu") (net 2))
 (segment (start 166.805 94.742) (end 167.752 94.742) (width 0.25) (layer "F.Cu") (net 2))
 (segment (start 162.88 95.8189) (end 165.728 95.8189) (width 0.25) (layer "F.Cu") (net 2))
 (segment (start 156.79 94.5729) (end 157.435 93.9283) (width 0.25) (layer "F.Cu") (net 2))
 (segment (start 152.405 95.758) (end 152.405 96.5849) (width 0.25) (layer "F.Cu") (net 2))
 (segment (start 167.752 94.862) (end 169.853 96.9631) (width 0.25) (layer "F.Cu") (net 2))
 (segment (start 157.435 93.9283) (end 162.643 93.9283) (width 0.25) (layer "F.Cu") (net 2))
 (segment (start 162.201 100.096) (end 161.451 100.096) (width 0.25) (layer "F.Cu") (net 2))
 (segment (start 154.778 96.5849) (end 156.79 94.5729) (width 0.25) (layer "F.Cu") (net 2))
 (segment (start 169.677 100.838) (end 169.677 99.7611) (width 0.25) (layer "F.Cu") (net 2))
 (segment (start 152.405 96.5849) (end 154.778 96.5849) (width 0.25) (layer "F.Cu") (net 2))
 (segment (start 161.451 100.096) (end 160.201 101.346) (width 0.25) (layer "F.Cu") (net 2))
 (segment (start 162.643 94.7552) (end 162.643 95.5821) (width 0.25) (layer "F.Cu") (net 2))
 (segment (start 169.853 96.9631) (end 169.853 97.79) (width 0.25) (layer "F.Cu") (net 2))
 (segment (start 142.929 104.394) (end 145.796 104.394) (width 0.25) (layer "B.Cu") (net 2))
 (segment (start 145.796 104.394) (end 145.796 93.8691) (width 0.25) (layer "B.Cu") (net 2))
 (segment (start 145.796 93.8691) (end 150.941 88.724) (width 0.25) (layer "B.Cu") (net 2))
 (segment (start 167.605 93.6651) (end 165.982 93.6651) (width 0.25) (layer "F.Cu") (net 1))
 (segment (start 142.929 106.934) (end 157.154 106.934) (width 0.25) (layer "F.Cu") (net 1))
 (segment (start 163.958 94.742) (end 163.958 94.5053) (width 0.25) (layer "F.Cu") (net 1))
 (segment (start 167.715 104.637) (end 170.731 101.6214) (width 0.25) (layer "F.Cu") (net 1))
 (segment (start 155.937 86.4839) (end 151.971 86.4839) (width 0.25) (layer "F.Cu") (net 1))
 (segment (start 170.731 101.6214) (end 170.731 96.7903) (width 0.25) (layer "F.Cu") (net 1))
 (segment (start 159.451 104.637) (end 159.451 103.346) (width 0.25) (layer "F.Cu") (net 1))
 (segment (start 151.971 86.4839) (end 151.841 86.614) (width 0.25) (layer "F.Cu") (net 1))
 (segment (start 166.83 100.838) (end 165.072 102.596) (width 0.25) (layer "F.Cu") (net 1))
 (segment (start 162.201 103.3553) (end 162.201 102.596) (width 0.25) (layer "F.Cu") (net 1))
 (segment (start 157.154 106.934) (end 159.451 104.637) (width 0.25) (layer "F.Cu") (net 1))
 (segment (start 164.905 94.742) (end 163.958 94.742) (width 0.25) (layer "F.Cu") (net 1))
 (segment (start 165.072 102.596) (end 162.201 102.596) (width 0.25) (layer "F.Cu") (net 1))
 (segment (start 159.451 104.637) (end 167.715 104.637) (width 0.25) (layer "F.Cu") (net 1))
 (segment (start 165.982 93.6651) (end 164.905 94.742) (width 0.25) (layer "F.Cu") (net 1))
 (segment (start 163.958 94.5053) (end 155.937 86.4839) (width 0.25) (layer "F.Cu") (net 1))
 (segment (start 170.731 96.7903) (end 167.605 93.6651) (width 0.25) (layer "F.Cu") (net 1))
 (segment (start 167.777 100.838) (end 166.83 100.838) (width 0.25) (layer "F.Cu") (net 1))
 (via (at 162.201 103.3553) (size 0.8) (drill 0.4) (layers "F.Cu" "B.Cu") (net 1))
 (segment (start 142.929 106.934) (end 158.622 106.934) (width 0.25) (layer "B.Cu") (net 1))
 (segment (start 158.622 106.934) (end 162.201 103.3553) (width 0.25) (layer "B.Cu") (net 1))
 (segment (start 154.105 95.758) (end 154.105 94.9311) (width 0.25) (layer "F.Cu") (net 17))
 (segment (start 154.105 94.9311) (end 149.79 90.6159) (width 0.25) (layer "F.Cu") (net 17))
 (segment (start 149.79 90.6159) (end 149.79 87.7152) (width 0.25) (layer "F.Cu") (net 17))
 (segment (start 149.79 87.7152) (end 150.041 87.464) (width 0.25) (layer "F.Cu") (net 17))
 (segment (start 168.724 99.1878) (end 168.724 101.7842) (width 0.25) (layer "F.Cu") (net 5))
 (segment (start 168.724 101.7842) (end 166.385 104.1231) (width 0.25) (layer "F.Cu") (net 5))
 (segment (start 168.153 98.6169) (end 168.724 99.1878) (width 0.25) (layer "F.Cu") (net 5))
 (segment (start 168.153 97.79) (end 168.153 98.6169) (width 0.25) (layer "F.Cu") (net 5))
 (segment (start 166.385 104.1231) (end 160.742 104.1231) (width 0.25) (layer "F.Cu") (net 5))
 (segment (start 160.742 104.1231) (end 160.451 103.8317) (width 0.25) (layer "F.Cu") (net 5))
 (segment (start 160.451 103.8317) (end 160.451 103.346) (width 0.25) (layer "F.Cu") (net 5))
 (segment (start 160.9434 95.1682) (end 160.9434 94.7552) (width 0.25) (layer "F.Cu") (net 25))
 (segment (start 160.943 95.5821) (end 160.951 95.5897) (width 0.25) (layer "F.Cu") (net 25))
 (segment (start 160.943 95.1686) (end 160.9434 95.1682) (width 0.25) (layer "F.Cu") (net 25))
 (segment (start 160.951 95.5897) (end 160.951 99.346) (width 0.25) (layer "F.Cu") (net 25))
 (segment (start 160.943 95.1686) (end 160.943 95.5821) (width 0.25) (layer "F.Cu") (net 25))
 (segment (start 160.943 94.7552) (end 160.943 95.1686) (width 0.25) (layer "F.Cu") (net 25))
 (segment (start 157.529 98.6188) (end 159.268 98.6188) (width 0.25) (layer "F.Cu") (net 28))
 (segment (start 159.268 98.6188) (end 159.451 98.8017) (width 0.25) (layer "F.Cu") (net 28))
 (segment (start 159.451 98.8017) (end 159.451 99.346) (width 0.25) (layer "F.Cu") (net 28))
 (segment (start 153.597 103.378) (end 153.597 102.5511) (width 0.25) (layer "F.Cu") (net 28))
 (segment (start 153.597 102.5511) (end 157.529 98.6188) (width 0.25) (layer "F.Cu") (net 28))
 (segment (start 158.951 99.346) (end 157.941 99.346) (width 0.25) (layer "F.Cu") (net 3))
 (segment (start 152.405 98.806) (end 152.405 97.9791) (width 0.25) (layer "F.Cu") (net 3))
 (segment (start 152.405 97.9791) (end 156.574 97.9791) (width 0.25) (layer "F.Cu") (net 3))
 (via (at 157.941 99.346) (size 0.8) (drill 0.4) (layers "F.Cu" "B.Cu") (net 3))
 (via (at 156.574 97.9791) (size 0.8) (drill 0.4) (layers "F.Cu" "B.Cu") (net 3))
 (segment (start 157.941 99.346) (end 156.574 97.9791) (width 0.25) (layer "B.Cu") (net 3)))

